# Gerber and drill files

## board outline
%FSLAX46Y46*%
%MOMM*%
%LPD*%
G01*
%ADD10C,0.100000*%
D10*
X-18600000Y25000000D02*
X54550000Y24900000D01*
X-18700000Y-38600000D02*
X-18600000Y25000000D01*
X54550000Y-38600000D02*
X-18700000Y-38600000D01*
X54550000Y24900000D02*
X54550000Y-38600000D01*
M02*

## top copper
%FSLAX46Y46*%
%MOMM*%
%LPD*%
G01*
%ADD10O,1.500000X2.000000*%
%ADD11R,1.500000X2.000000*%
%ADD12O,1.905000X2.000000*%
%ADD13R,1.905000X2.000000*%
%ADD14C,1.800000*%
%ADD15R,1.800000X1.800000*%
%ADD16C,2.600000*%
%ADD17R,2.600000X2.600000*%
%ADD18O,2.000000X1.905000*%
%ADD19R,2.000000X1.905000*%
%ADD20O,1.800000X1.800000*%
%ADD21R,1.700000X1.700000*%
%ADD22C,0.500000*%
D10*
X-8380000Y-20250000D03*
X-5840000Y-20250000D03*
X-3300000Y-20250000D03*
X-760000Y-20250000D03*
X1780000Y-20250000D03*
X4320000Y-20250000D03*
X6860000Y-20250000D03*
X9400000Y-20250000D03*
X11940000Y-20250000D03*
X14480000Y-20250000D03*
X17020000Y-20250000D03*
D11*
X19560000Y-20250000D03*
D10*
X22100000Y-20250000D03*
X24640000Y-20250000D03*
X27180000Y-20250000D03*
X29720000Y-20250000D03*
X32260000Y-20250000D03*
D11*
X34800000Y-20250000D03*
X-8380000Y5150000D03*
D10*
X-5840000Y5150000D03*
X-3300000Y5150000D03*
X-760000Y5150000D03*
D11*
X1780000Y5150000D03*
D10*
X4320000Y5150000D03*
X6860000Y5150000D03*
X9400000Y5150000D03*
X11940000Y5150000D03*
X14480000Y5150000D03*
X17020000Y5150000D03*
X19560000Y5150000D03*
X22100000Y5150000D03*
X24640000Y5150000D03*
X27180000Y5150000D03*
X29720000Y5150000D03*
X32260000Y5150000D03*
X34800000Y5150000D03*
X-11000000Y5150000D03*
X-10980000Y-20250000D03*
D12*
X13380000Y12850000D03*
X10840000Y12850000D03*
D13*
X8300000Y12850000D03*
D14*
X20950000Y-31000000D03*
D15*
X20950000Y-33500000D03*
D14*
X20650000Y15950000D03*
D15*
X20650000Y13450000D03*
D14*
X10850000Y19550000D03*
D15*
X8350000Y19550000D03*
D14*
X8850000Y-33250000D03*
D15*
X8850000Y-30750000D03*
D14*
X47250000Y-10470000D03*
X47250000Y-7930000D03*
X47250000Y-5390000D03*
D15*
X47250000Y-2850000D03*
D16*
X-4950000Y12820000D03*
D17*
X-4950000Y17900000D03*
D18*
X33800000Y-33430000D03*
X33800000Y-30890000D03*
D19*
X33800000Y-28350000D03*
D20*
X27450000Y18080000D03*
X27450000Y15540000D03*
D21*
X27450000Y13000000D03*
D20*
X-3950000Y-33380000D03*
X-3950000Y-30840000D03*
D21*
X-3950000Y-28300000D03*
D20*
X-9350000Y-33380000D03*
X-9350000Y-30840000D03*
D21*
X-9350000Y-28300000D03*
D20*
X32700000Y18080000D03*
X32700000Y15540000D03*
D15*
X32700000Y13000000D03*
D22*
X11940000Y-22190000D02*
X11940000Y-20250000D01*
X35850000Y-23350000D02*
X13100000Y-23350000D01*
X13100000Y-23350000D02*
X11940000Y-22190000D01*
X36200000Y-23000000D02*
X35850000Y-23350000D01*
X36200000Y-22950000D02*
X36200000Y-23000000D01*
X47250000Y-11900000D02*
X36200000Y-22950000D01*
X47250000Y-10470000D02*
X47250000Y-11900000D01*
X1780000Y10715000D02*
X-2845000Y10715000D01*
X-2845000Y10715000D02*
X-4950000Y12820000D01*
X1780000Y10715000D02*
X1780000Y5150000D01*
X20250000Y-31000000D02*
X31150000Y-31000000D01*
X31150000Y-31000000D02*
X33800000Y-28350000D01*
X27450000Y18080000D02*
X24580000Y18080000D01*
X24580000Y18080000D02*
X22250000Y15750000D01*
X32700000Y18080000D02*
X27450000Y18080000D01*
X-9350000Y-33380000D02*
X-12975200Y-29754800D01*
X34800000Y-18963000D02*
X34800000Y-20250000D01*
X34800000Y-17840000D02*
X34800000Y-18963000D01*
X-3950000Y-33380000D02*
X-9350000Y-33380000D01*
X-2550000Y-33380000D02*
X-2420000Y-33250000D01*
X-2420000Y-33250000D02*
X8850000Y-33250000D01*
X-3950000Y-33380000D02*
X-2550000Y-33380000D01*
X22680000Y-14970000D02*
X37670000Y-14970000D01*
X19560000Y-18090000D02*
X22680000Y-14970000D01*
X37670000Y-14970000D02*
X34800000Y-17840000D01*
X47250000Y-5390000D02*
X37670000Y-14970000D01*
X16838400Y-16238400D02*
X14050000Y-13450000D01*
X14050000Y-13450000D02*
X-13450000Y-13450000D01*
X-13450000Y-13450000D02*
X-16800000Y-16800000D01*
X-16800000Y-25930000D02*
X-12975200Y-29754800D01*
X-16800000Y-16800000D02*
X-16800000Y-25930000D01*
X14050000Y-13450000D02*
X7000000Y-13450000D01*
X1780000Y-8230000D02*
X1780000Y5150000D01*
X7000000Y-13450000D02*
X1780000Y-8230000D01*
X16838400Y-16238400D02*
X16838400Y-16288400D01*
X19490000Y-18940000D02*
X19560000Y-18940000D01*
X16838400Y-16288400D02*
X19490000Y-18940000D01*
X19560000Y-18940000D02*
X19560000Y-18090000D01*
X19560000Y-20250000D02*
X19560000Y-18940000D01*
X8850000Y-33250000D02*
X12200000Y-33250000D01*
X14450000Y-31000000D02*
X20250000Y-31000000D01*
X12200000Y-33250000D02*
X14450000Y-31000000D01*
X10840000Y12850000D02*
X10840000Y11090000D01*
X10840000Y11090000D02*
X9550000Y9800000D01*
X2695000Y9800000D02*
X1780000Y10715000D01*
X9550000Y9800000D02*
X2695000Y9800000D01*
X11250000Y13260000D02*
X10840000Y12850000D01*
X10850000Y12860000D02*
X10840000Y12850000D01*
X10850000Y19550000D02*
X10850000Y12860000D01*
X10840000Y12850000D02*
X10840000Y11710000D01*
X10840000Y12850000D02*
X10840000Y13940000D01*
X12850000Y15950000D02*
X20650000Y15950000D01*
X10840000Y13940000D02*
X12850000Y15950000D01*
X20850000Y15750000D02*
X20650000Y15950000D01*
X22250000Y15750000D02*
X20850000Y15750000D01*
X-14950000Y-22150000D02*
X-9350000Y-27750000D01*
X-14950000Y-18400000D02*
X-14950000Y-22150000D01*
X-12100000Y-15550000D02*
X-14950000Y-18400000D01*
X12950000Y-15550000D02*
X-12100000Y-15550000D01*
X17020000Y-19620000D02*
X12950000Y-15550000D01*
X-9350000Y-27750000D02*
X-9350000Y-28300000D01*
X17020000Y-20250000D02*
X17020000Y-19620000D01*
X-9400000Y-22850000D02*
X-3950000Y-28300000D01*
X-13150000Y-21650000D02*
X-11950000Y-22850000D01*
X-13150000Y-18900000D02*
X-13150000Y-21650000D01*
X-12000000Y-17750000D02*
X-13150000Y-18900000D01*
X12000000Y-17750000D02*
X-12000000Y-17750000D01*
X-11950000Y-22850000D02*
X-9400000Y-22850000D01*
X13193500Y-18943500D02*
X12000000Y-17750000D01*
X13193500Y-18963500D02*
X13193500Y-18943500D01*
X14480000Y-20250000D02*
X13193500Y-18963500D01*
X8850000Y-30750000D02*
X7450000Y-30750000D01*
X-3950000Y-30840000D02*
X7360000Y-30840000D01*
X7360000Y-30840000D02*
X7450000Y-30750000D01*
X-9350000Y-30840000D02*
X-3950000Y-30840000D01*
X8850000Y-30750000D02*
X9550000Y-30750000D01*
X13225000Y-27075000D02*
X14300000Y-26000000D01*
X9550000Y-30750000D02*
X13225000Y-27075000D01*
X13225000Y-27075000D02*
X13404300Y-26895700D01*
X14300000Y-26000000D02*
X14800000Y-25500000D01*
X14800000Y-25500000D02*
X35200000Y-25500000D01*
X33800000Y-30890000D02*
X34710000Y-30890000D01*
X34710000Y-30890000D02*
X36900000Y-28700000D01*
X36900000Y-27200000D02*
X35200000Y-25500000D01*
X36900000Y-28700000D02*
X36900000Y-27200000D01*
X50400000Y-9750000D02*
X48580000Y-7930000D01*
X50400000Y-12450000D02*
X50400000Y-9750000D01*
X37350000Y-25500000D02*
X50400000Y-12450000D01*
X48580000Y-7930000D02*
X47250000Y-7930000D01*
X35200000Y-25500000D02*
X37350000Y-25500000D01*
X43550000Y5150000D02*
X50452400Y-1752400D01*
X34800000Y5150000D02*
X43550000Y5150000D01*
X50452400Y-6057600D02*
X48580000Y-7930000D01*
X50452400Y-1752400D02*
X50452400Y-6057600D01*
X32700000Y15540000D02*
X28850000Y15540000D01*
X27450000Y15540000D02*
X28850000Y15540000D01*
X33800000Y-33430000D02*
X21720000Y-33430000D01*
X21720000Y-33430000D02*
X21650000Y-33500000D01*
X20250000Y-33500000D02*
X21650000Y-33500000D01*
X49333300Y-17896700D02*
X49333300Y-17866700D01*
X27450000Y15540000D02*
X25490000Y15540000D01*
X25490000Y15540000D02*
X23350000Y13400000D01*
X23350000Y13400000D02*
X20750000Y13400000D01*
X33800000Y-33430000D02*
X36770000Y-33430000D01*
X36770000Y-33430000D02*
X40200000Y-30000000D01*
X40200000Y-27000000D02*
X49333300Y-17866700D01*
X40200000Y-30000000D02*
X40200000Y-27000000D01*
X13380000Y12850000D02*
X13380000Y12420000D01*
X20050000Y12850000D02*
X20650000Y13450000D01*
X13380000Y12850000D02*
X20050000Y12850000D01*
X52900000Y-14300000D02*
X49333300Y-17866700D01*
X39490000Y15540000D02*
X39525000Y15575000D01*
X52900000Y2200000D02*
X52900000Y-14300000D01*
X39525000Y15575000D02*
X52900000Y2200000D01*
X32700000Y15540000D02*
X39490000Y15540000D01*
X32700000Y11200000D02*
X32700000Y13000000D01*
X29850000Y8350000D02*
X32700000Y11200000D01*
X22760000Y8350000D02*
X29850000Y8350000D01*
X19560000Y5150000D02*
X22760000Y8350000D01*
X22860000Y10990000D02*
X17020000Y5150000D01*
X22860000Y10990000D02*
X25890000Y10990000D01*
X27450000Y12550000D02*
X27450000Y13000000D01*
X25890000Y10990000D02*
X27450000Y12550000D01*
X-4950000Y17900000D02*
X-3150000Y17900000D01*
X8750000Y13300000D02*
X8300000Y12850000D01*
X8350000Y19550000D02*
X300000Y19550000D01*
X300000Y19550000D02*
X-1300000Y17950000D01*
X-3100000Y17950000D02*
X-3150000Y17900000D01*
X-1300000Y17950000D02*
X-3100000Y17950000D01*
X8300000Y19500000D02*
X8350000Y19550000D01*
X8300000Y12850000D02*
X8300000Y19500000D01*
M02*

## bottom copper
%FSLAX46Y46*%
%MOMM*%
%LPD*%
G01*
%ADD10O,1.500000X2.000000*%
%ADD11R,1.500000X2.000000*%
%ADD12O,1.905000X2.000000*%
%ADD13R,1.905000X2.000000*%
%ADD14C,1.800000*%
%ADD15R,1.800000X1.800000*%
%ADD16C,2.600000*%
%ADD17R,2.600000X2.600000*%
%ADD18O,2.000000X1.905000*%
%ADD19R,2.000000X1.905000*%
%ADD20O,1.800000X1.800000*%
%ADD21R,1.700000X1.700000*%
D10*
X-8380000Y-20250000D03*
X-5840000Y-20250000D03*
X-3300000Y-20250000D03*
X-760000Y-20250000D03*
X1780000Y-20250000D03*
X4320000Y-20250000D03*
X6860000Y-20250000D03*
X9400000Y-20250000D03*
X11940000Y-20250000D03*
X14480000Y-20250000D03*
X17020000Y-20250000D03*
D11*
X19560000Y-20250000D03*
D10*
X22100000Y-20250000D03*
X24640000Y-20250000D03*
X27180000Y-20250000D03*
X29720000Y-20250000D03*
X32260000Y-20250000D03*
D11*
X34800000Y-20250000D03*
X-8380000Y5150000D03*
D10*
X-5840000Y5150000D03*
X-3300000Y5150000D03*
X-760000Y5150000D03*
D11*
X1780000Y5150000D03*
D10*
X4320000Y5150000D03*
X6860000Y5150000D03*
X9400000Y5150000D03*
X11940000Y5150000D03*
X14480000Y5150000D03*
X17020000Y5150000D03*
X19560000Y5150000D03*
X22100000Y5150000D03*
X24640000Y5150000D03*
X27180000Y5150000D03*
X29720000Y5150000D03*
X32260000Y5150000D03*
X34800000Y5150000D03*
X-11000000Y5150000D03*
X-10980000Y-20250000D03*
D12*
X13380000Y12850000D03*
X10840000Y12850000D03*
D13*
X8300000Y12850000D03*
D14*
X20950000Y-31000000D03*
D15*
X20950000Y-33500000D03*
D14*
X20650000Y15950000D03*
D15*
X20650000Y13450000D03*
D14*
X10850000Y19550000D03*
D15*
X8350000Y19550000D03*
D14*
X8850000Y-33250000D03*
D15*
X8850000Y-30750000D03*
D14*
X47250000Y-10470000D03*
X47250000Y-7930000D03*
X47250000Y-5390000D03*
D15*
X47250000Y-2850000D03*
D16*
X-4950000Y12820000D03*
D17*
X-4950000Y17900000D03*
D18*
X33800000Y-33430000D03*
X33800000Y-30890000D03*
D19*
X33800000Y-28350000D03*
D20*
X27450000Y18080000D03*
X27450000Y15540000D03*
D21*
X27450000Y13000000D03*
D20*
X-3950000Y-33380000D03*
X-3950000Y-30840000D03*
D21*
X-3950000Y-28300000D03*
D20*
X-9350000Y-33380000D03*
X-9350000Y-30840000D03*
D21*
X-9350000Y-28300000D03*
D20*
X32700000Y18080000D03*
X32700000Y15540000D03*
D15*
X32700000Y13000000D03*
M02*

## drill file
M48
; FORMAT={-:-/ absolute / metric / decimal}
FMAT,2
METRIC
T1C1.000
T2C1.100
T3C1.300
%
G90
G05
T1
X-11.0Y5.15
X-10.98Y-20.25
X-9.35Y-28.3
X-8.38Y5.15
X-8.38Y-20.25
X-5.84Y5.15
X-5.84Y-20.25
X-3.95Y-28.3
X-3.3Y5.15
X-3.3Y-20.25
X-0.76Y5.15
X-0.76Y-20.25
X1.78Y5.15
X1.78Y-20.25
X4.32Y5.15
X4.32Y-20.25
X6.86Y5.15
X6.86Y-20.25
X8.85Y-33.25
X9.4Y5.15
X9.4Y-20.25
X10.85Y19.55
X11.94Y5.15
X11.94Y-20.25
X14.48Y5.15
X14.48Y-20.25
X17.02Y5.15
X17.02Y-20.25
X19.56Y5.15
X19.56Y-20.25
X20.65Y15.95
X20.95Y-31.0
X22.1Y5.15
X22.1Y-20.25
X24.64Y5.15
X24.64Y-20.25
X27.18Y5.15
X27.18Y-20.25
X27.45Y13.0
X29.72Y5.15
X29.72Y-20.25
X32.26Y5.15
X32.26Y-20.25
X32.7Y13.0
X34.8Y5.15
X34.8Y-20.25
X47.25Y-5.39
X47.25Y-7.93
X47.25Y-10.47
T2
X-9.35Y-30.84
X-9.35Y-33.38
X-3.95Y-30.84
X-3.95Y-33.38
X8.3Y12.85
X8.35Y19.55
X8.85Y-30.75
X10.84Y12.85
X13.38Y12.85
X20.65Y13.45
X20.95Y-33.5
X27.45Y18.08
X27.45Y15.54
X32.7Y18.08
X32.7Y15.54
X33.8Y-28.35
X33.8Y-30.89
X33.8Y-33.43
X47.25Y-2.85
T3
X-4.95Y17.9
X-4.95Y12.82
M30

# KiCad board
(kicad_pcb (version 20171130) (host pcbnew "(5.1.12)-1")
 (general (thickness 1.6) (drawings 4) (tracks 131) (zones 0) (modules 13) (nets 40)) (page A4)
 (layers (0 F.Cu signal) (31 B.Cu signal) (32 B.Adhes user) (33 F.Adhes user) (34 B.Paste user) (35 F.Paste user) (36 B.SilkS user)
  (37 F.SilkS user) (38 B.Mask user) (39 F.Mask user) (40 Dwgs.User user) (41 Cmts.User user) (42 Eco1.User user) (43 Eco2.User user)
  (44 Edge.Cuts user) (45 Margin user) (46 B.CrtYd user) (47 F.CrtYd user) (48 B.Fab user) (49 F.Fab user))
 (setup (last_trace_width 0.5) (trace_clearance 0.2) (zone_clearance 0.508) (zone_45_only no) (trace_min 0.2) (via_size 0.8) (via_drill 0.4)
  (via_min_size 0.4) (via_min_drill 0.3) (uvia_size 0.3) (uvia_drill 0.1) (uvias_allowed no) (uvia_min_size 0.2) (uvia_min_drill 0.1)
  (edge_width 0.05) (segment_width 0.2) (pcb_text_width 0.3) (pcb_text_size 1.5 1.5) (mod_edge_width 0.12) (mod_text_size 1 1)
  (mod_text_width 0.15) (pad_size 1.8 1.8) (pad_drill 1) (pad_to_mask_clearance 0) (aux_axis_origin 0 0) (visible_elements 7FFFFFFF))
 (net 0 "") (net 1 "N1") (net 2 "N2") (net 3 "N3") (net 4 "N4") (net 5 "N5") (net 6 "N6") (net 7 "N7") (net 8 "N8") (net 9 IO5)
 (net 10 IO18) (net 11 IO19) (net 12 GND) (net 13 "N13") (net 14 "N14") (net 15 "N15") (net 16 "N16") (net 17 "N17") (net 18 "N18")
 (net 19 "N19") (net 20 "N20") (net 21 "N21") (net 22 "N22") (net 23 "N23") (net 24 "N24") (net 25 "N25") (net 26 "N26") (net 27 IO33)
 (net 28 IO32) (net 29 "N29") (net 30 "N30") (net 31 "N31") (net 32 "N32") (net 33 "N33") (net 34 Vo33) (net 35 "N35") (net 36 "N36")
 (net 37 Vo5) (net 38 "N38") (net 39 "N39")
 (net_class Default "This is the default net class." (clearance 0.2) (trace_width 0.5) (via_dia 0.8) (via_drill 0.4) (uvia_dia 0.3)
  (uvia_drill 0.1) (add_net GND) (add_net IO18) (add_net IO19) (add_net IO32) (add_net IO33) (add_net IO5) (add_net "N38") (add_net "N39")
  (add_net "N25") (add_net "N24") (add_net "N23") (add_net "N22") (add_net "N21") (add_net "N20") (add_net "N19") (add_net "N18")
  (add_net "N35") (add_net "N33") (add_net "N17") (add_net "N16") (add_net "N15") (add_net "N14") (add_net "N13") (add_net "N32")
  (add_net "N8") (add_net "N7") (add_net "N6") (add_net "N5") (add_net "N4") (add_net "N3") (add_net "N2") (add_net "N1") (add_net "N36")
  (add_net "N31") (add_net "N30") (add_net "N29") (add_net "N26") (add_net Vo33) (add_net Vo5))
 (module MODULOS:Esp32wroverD (layer F.Cu) (at 12.4 7.55)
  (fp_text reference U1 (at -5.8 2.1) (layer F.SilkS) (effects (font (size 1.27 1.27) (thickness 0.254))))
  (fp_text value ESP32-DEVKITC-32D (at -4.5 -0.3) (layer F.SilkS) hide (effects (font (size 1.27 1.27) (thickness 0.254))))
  (pad 37 thru_hole oval (at -20.78 12.7) (size 1.5 2) (drill 1) (layers *.Cu *.Mask) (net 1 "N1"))
  (pad 36 thru_hole oval (at -18.24 12.7) (size 1.5 2) (drill 1) (layers *.Cu *.Mask) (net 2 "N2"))
  (pad 35 thru_hole oval (at -15.7 12.7) (size 1.5 2) (drill 1) (layers *.Cu *.Mask) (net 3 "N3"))
  (pad 34 thru_hole oval (at -13.16 12.7) (size 1.5 2) (drill 1) (layers *.Cu *.Mask) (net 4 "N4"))
  (pad 33 thru_hole oval (at -10.62 12.7) (size 1.5 2) (drill 1) (layers *.Cu *.Mask) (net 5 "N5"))
  (pad 32 thru_hole oval (at -8.08 12.7) (size 1.5 2) (drill 1) (layers *.Cu *.Mask) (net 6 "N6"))
  (pad 31 thru_hole oval (at -5.54 12.7) (size 1.5 2) (drill 1) (layers *.Cu *.Mask) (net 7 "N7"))
  (pad 30 thru_hole oval (at -3 12.7) (size 1.5 2) (drill 1) (layers *.Cu *.Mask) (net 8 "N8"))
  (pad 29 thru_hole oval (at -0.46 12.7) (size 1.5 2) (drill 1) (layers *.Cu *.Mask) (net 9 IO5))
  (pad 28 thru_hole oval (at 2.08 12.7) (size 1.5 2) (drill 1) (layers *.Cu *.Mask) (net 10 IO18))
  (pad 27 thru_hole oval (at 4.62 12.7) (size 1.5 2) (drill 1) (layers *.Cu *.Mask) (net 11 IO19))
  (pad 26 thru_hole rect (at 7.16 12.7) (size 1.5 2) (drill 1) (layers *.Cu *.Mask) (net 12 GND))
  (pad 25 thru_hole oval (at 9.7 12.7) (size 1.5 2) (drill 1) (layers *.Cu *.Mask) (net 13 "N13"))
  (pad 24 thru_hole oval (at 12.24 12.7) (size 1.5 2) (drill 1) (layers *.Cu *.Mask) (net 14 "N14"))
  (pad 23 thru_hole oval (at 14.78 12.7) (size 1.5 2) (drill 1) (layers *.Cu *.Mask) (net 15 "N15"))
  (pad 22 thru_hole oval (at 17.32 12.7) (size 1.5 2) (drill 1) (layers *.Cu *.Mask) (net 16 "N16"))
  (pad 21 thru_hole oval (at 19.86 12.7) (size 1.5 2) (drill 1) (layers *.Cu *.Mask) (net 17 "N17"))
  (pad 20 thru_hole rect (at 22.4 12.7) (size 1.5 2) (drill 1) (layers *.Cu *.Mask) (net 12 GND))
  (pad 18 thru_hole rect (at -20.78 -12.7) (size 1.5 2) (drill 1) (layers *.Cu *.Mask) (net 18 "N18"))
  (pad 17 thru_hole oval (at -18.24 -12.7) (size 1.5 2) (drill 1) (layers *.Cu *.Mask) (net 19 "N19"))
  (pad 16 thru_hole oval (at -15.7 -12.7) (size 1.5 2) (drill 1) (layers *.Cu *.Mask) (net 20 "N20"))
  (pad 15 thru_hole oval (at -13.16 -12.7) (size 1.5 2) (drill 1) (layers *.Cu *.Mask) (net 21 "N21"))
  (pad 14 thru_hole rect (at -10.62 -12.7) (size 1.5 2) (drill 1) (layers *.Cu *.Mask) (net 12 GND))
  (pad 13 thru_hole oval (at -8.08 -12.7) (size 1.5 2) (drill 1) (layers *.Cu *.Mask) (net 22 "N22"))
  (pad 12 thru_hole oval (at -5.54 -12.7) (size 1.5 2) (drill 1) (layers *.Cu *.Mask) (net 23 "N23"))
  (pad 11 thru_hole oval (at -3 -12.7) (size 1.5 2) (drill 1) (layers *.Cu *.Mask) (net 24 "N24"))
  (pad 10 thru_hole oval (at -0.46 -12.7) (size 1.5 2) (drill 1) (layers *.Cu *.Mask) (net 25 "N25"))
  (pad 9 thru_hole oval (at 2.08 -12.7) (size 1.5 2) (drill 1) (layers *.Cu *.Mask) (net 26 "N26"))
  (pad 8 thru_hole oval (at 4.62 -12.7) (size 1.5 2) (drill 1) (layers *.Cu *.Mask) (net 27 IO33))
  (pad 7 thru_hole oval (at 7.16 -12.7) (size 1.5 2) (drill 1) (layers *.Cu *.Mask) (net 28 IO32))
  (pad 6 thru_hole oval (at 9.7 -12.7) (size 1.5 2) (drill 1) (layers *.Cu *.Mask) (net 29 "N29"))
  (pad 5 thru_hole oval (at 12.24 -12.7) (size 1.5 2) (drill 1) (layers *.Cu *.Mask) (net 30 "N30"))
  (pad 4 thru_hole oval (at 14.78 -12.7) (size 1.5 2) (drill 1) (layers *.Cu *.Mask) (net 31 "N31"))
  (pad 3 thru_hole oval (at 17.32 -12.7) (size 1.5 2) (drill 1) (layers *.Cu *.Mask) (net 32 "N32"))
  (pad 2 thru_hole oval (at 19.86 -12.7) (size 1.5 2) (drill 1) (layers *.Cu *.Mask) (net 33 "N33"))
  (pad 1 thru_hole oval (at 22.4 -12.7) (size 1.5 2) (drill 1) (layers *.Cu *.Mask) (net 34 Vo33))
  (pad 19 thru_hole oval (at -23.4 -12.7) (size 1.5 2) (drill 1) (layers *.Cu *.Mask) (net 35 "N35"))
  (pad 38 thru_hole oval (at -23.38 12.7) (size 1.5 2) (drill 1) (layers *.Cu *.Mask) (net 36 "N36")))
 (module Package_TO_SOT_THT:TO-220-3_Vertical (layer F.Cu) (at 8.3 -12.85)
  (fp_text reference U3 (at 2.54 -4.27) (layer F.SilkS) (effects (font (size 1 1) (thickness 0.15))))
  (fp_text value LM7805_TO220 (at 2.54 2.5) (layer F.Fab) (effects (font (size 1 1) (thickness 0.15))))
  (pad 3 thru_hole oval (at 5.08 0) (size 1.905 2) (drill 1.1) (layers *.Cu *.Mask) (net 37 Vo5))
  (pad 2 thru_hole oval (at 2.54 0) (size 1.905 2) (drill 1.1) (layers *.Cu *.Mask) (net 12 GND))
  (pad 1 thru_hole rect (at 0 0) (size 1.905 2) (drill 1.1) (layers *.Cu *.Mask) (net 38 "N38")))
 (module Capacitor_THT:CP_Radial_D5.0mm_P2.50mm (layer F.Cu) (at 20.95 33.5 90)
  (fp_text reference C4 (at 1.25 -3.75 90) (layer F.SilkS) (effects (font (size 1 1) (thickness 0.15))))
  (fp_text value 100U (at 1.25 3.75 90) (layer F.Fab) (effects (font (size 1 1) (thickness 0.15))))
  (pad 2 thru_hole circle (at 2.5 0 90) (size 1.8 1.8) (drill 1) (layers *.Cu *.Mask) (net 12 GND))
  (pad 1 thru_hole rect (at 0 0 90) (size 1.8 1.8) (drill 1.1) (layers *.Cu *.Mask) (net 37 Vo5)))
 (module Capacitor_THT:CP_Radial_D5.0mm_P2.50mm (layer F.Cu) (at 20.65 -13.45 90)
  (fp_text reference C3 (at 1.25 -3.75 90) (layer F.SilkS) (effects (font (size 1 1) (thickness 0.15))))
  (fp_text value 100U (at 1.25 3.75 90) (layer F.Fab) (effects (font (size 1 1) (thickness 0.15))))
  (pad 2 thru_hole circle (at 2.5 0 90) (size 1.8 1.8) (drill 1) (layers *.Cu *.Mask) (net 12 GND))
  (pad 1 thru_hole rect (at 0 0 90) (size 1.8 1.8) (drill 1.1) (layers *.Cu *.Mask) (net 37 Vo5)))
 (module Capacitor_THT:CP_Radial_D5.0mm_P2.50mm (layer F.Cu) (at 8.35 -19.55)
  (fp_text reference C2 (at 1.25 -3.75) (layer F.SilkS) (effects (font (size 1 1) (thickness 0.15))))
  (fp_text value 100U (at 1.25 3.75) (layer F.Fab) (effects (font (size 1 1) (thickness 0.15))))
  (pad 2 thru_hole circle (at 2.5 0) (size 1.8 1.8) (drill 1) (layers *.Cu *.Mask) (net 12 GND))
  (pad 1 thru_hole rect (at 0 0) (size 1.8 1.8) (drill 1.1) (layers *.Cu *.Mask) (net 38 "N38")))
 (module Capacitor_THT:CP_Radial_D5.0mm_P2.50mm (layer F.Cu) (at 8.85 30.75 270)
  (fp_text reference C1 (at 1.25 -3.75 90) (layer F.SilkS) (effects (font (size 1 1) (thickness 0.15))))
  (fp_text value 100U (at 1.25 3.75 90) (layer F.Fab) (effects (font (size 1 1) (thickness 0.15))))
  (pad 2 thru_hole circle (at 2.5 0 270) (size 1.8 1.8) (drill 1) (layers *.Cu *.Mask) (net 12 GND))
  (pad 1 thru_hole rect (at 0 0 270) (size 1.8 1.8) (drill 1.1) (layers *.Cu *.Mask) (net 34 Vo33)))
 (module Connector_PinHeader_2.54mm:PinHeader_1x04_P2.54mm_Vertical (layer F.Cu) (at 47.25 2.85)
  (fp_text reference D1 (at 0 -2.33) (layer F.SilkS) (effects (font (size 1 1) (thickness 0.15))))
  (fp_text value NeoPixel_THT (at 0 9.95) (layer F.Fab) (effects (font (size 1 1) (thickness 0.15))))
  (pad 4 thru_hole circle (at 0 7.62) (size 1.8 1.8) (drill 1) (layers *.Cu *.Mask) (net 9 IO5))
  (pad 3 thru_hole circle (at 0 5.08) (size 1.8 1.8) (drill 1) (layers *.Cu *.Mask) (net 34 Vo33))
  (pad 2 thru_hole circle (at 0 2.54) (size 1.8 1.8) (drill 1) (layers *.Cu *.Mask) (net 12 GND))
  (pad 1 thru_hole rect (at 0 0) (size 1.8 1.8) (drill 1.1) (layers *.Cu *.Mask) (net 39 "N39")))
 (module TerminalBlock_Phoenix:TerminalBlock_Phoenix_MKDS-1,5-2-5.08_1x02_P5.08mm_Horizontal (layer F.Cu) (at -4.95 -17.9 270)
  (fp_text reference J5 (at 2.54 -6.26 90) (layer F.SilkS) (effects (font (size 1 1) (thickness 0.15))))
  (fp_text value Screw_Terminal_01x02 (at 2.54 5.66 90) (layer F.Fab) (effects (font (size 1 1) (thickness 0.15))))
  (pad 2 thru_hole circle (at 5.08 0 270) (size 2.6 2.6) (drill 1.3) (layers *.Cu *.Mask) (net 12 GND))
  (pad 1 thru_hole rect (at 0 0 270) (size 2.6 2.6) (drill 1.3) (layers *.Cu *.Mask) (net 38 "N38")))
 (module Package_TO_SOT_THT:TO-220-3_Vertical (layer F.Cu) (at 33.8 28.35 270)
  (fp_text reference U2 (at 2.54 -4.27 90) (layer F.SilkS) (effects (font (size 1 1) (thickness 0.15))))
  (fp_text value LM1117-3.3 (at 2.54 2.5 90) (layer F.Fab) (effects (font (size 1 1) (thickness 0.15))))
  (pad 3 thru_hole oval (at 5.08 0 270) (size 1.905 2) (drill 1.1) (layers *.Cu *.Mask) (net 37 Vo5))
  (pad 2 thru_hole oval (at 2.54 0 270) (size 1.905 2) (drill 1.1) (layers *.Cu *.Mask) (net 34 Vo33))
  (pad 1 thru_hole rect (at 0 0 270) (size 1.905 2) (drill 1.1) (layers *.Cu *.Mask) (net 12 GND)))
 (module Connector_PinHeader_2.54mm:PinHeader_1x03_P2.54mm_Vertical (layer F.Cu) (at 27.45 -13 180)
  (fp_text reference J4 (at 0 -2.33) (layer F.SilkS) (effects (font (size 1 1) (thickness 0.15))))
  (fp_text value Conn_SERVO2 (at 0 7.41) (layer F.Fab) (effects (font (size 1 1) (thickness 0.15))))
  (pad 3 thru_hole oval (at 0 5.08 180) (size 1.8 1.8) (drill 1.1) (layers *.Cu *.Mask) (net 12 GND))
  (pad 2 thru_hole oval (at 0 2.54 180) (size 1.8 1.8) (drill 1.1) (layers *.Cu *.Mask) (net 37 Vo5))
  (pad 1 thru_hole rect (at 0 0 180) (size 1.7 1.7) (drill 1) (layers *.Cu *.Mask) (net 27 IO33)))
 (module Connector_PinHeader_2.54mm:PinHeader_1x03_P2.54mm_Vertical (layer F.Cu) (at -3.95 28.3)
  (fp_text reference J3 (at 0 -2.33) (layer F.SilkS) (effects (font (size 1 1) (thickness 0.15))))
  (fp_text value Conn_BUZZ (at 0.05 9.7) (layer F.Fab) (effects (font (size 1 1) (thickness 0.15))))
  (pad 3 thru_hole oval (at 0 5.08) (size 1.8 1.8) (drill 1.1) (layers *.Cu *.Mask) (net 12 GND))
  (pad 2 thru_hole oval (at 0 2.54) (size 1.8 1.8) (drill 1.1) (layers *.Cu *.Mask) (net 34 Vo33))
  (pad 1 thru_hole rect (at 0 0) (size 1.7 1.7) (drill 1) (layers *.Cu *.Mask) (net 10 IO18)))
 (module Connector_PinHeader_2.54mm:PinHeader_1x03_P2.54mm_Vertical (layer F.Cu) (at -9.35 28.3)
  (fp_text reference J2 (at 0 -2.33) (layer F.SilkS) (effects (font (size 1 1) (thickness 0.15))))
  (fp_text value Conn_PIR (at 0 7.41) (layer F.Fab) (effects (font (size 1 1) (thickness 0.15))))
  (pad 3 thru_hole oval (at 0 5.08) (size 1.8 1.8) (drill 1.1) (layers *.Cu *.Mask) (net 12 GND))
  (pad 2 thru_hole oval (at 0 2.54) (size 1.8 1.8) (drill 1.1) (layers *.Cu *.Mask) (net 34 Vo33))
  (pad 1 thru_hole rect (at 0 0) (size 1.7 1.7) (drill 1) (layers *.Cu *.Mask) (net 11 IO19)))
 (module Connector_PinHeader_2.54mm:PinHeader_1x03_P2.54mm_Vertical (layer F.Cu) (at 32.7 -13 180)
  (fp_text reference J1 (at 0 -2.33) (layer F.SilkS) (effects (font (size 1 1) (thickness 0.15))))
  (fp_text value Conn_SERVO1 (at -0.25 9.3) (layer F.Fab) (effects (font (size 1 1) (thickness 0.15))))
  (pad 3 thru_hole oval (at 0 5.08 180) (size 1.8 1.8) (drill 1.1) (layers *.Cu *.Mask) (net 12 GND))
  (pad 2 thru_hole oval (at 0 2.54 180) (size 1.8 1.8) (drill 1.1) (layers *.Cu *.Mask) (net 37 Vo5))
  (pad 1 thru_hole rect (at 0 0 180) (size 1.8 1.8) (drill 1) (layers *.Cu *.Mask) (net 28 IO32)))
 (gr_line (start -18.6 -25) (end 54.55 -24.9) (layer Edge.Cuts) (width 0.1))
 (gr_line (start -18.7 38.6) (end -18.6 -25) (layer Edge.Cuts) (width 0.1))
 (gr_line (start 54.55 38.6) (end -18.7 38.6) (layer Edge.Cuts) (width 0.1))
 (gr_line (start 54.55 -24.9) (end 54.55 38.6) (layer Edge.Cuts) (width 0.1))
 (segment (start 11.94 22.19) (end 11.94 20.25) (width 0.5) (layer F.Cu) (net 9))
 (segment (start 35.85 23.35) (end 13.1 23.35) (width 0.5) (layer F.Cu) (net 9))
 (segment (start 13.1 23.35) (end 11.94 22.19) (width 0.5) (layer F.Cu) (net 9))
 (segment (start 36.2 23) (end 35.85 23.35) (width 0.5) (layer F.Cu) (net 9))
 (segment (start 36.2 22.95) (end 36.2 23) (width 0.5) (layer F.Cu) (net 9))
 (segment (start 47.25 11.9) (end 36.2 22.95) (width 0.5) (layer F.Cu) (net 9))
 (segment (start 47.25 10.47) (end 47.25 11.9) (width 0.5) (layer F.Cu) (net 9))
 (segment (start 1.78 -10.715) (end -2.845 -10.715) (width 0.5) (layer F.Cu) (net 12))
 (segment (start -2.845 -10.715) (end -4.95 -12.82) (width 0.5) (layer F.Cu) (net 12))
 (segment (start 1.78 -10.715) (end 1.78 -5.15) (width 0.5) (layer F.Cu) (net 12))
 (segment (start 20.25 31) (end 31.15 31) (width 0.5) (layer F.Cu) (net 12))
 (segment (start 31.15 31) (end 33.8 28.35) (width 0.5) (layer F.Cu) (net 12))
 (segment (start 27.45 -18.08) (end 24.58 -18.08) (width 0.5) (layer F.Cu) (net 12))
 (segment (start 24.58 -18.08) (end 22.25 -15.75) (width 0.5) (layer F.Cu) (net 12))
 (segment (start 32.7 -18.08) (end 27.45 -18.08) (width 0.5) (layer F.Cu) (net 12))
 (segment (start -9.35 33.38) (end -12.9752 29.7548) (width 0.5) (layer F.Cu) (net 12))
 (segment (start 34.8 18.963) (end 34.8 20.25) (width 0.5) (layer F.Cu) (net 12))
 (segment (start 34.8 17.84) (end 34.8 18.963) (width 0.5) (layer F.Cu) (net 12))
 (segment (start -3.95 33.38) (end -9.35 33.38) (width 0.5) (layer F.Cu) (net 12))
 (segment (start -2.55 33.38) (end -2.42 33.25) (width 0.5) (layer F.Cu) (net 12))
 (segment (start -2.42 33.25) (end 8.85 33.25) (width 0.5) (layer F.Cu) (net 12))
 (segment (start -3.95 33.38) (end -2.55 33.38) (width 0.5) (layer F.Cu) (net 12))
 (segment (start 22.68 14.97) (end 37.67 14.97) (width 0.5) (layer F.Cu) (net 12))
 (segment (start 19.56 18.09) (end 22.68 14.97) (width 0.5) (layer F.Cu) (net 12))
 (segment (start 37.67 14.97) (end 34.8 17.84) (width 0.5) (layer F.Cu) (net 12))
 (segment (start 47.25 5.39) (end 37.67 14.97) (width 0.5) (layer F.Cu) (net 12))
 (segment (start 16.8384 16.2384) (end 14.05 13.45) (width 0.5) (layer F.Cu) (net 12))
 (segment (start 14.05 13.45) (end -13.45 13.45) (width 0.5) (layer F.Cu) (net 12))
 (segment (start -13.45 13.45) (end -16.8 16.8) (width 0.5) (layer F.Cu) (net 12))
 (segment (start -16.8 25.93) (end -12.9752 29.7548) (width 0.5) (layer F.Cu) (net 12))
 (segment (start -16.8 16.8) (end -16.8 25.93) (width 0.5) (layer F.Cu) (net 12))
 (segment (start 14.05 13.45) (end 7 13.45) (width 0.5) (layer F.Cu) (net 12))
 (segment (start 1.78 8.23) (end 1.78 -5.15) (width 0.5) (layer F.Cu) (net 12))
 (segment (start 7 13.45) (end 1.78 8.23) (width 0.5) (layer F.Cu) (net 12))
 (segment (start 16.8384 16.2384) (end 16.8384 16.2884) (width 0.5) (layer F.Cu) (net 12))
 (segment (start 19.49 18.94) (end 19.56 18.94) (width 0.5) (layer F.Cu) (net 12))
 (segment (start 16.8384 16.2884) (end 19.49 18.94) (width 0.5) (layer F.Cu) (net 12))
 (segment (start 19.56 18.94) (end 19.56 18.09) (width 0.5) (layer F.Cu) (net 12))
 (segment (start 19.56 20.25) (end 19.56 18.94) (width 0.5) (layer F.Cu) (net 12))
 (segment (start 8.85 33.25) (end 12.2 33.25) (width 0.5) (layer F.Cu) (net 12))
 (segment (start 14.45 31) (end 20.25 31) (width 0.5) (layer F.Cu) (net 12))
 (segment (start 12.2 33.25) (end 14.45 31) (width 0.5) (layer F.Cu) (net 12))
 (segment (start 10.84 -12.85) (end 10.84 -11.09) (width 0.5) (layer F.Cu) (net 12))
 (segment (start 10.84 -11.09) (end 9.55 -9.8) (width 0.5) (layer F.Cu) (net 12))
 (segment (start 2.695 -9.8) (end 1.78 -10.715) (width 0.5) (layer F.Cu) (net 12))
 (segment (start 9.55 -9.8) (end 2.695 -9.8) (width 0.5) (layer F.Cu) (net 12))
 (segment (start 11.25 -13.26) (end 10.84 -12.85) (width 0.5) (layer F.Cu) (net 12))
 (segment (start 10.85 -12.86) (end 10.84 -12.85) (width 0.5) (layer F.Cu) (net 12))
 (segment (start 10.85 -19.55) (end 10.85 -12.86) (width 0.5) (layer F.Cu) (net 12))
 (segment (start 10.84 -12.85) (end 10.84 -11.71) (width 0.5) (layer F.Cu) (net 12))
 (segment (start 10.84 -12.85) (end 10.84 -13.94) (width 0.5) (layer F.Cu) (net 12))
 (segment (start 12.85 -15.95) (end 20.65 -15.95) (width 0.5) (layer F.Cu) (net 12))
 (segment (start 10.84 -13.94) (end 12.85 -15.95) (width 0.5) (layer F.Cu) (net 12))
 (segment (start 20.85 -15.75) (end 20.65 -15.95) (width 0.5) (layer F.Cu) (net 12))
 (segment (start 22.25 -15.75) (end 20.85 -15.75) (width 0.5) (layer F.Cu) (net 12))
 (segment (start -14.95 22.15) (end -9.35 27.75) (width 0.5) (layer F.Cu) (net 11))
 (segment (start -14.95 18.4) (end -14.95 22.15) (width 0.5) (layer F.Cu) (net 11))
 (segment (start -12.1 15.55) (end -14.95 18.4) (width 0.5) (layer F.Cu) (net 11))
 (segment (start 12.95 15.55) (end -12.1 15.55) (width 0.5) (layer F.Cu) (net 11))
 (segment (start 17.02 19.62) (end 12.95 15.55) (width 0.5) (layer F.Cu) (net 11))
 (segment (start -9.35 27.75) (end -9.35 28.3) (width 0.5) (layer F.Cu) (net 11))
 (segment (start 17.02 20.25) (end 17.02 19.62) (width 0.5) (layer F.Cu) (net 11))
 (segment (start -9.4 22.85) (end -3.95 28.3) (width 0.5) (layer F.Cu) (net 10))
 (segment (start -13.15 21.65) (end -11.95 22.85) (width 0.5) (layer F.Cu) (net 10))
 (segment (start -13.15 18.9) (end -13.15 21.65) (width 0.5) (layer F.Cu) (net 10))
 (segment (start -12 17.75) (end -13.15 18.9) (width 0.5) (layer F.Cu) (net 10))
 (segment (start 12 17.75) (end -12 17.75) (width 0.5) (layer F.Cu) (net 10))
 (segment (start -11.95 22.85) (end -9.4 22.85) (width 0.5) (layer F.Cu) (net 10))
 (segment (start 13.1935 18.9435) (end 12 17.75) (width 0.5) (layer F.Cu) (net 10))
 (segment (start 13.1935 18.9635) (end 13.1935 18.9435) (width 0.5) (layer F.Cu) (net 10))
 (segment (start 14.48 20.25) (end 13.1935 18.9635) (width 0.5) (layer F.Cu) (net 10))
 (segment (start 8.85 30.75) (end 7.45 30.75) (width 0.5) (layer F.Cu) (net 34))
 (segment (start -3.95 30.84) (end 7.36 30.84) (width 0.5) (layer F.Cu) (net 34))
 (segment (start 7.36 30.84) (end 7.45 30.75) (width 0.5) (layer F.Cu) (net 34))
 (segment (start -9.35 30.84) (end -3.95 30.84) (width 0.5) (layer F.Cu) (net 34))
 (segment (start 8.85 30.75) (end 9.55 30.75) (width 0.5) (layer F.Cu) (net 34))
 (segment (start 13.225 27.075) (end 14.3 26) (width 0.5) (layer F.Cu) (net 34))
 (segment (start 9.55 30.75) (end 13.225 27.075) (width 0.5) (layer F.Cu) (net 34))
 (segment (start 13.225 27.075) (end 13.4043 26.8957) (width 0.5) (layer F.Cu) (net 34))
 (segment (start 14.3 26) (end 14.8 25.5) (width 0.5) (layer F.Cu) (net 34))
 (segment (start 14.8 25.5) (end 35.2 25.5) (width 0.5) (layer F.Cu) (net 34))
 (segment (start 33.8 30.89) (end 34.71 30.89) (width 0.5) (layer F.Cu) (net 34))
 (segment (start 34.71 30.89) (end 36.9 28.7) (width 0.5) (layer F.Cu) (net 34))
 (segment (start 36.9 27.2) (end 35.2 25.5) (width 0.5) (layer F.Cu) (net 34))
 (segment (start 36.9 28.7) (end 36.9 27.2) (width 0.5) (layer F.Cu) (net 34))
 (segment (start 50.4 9.75) (end 48.58 7.93) (width 0.5) (layer F.Cu) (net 34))
 (segment (start 50.4 12.45) (end 50.4 9.75) (width 0.5) (layer F.Cu) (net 34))
 (segment (start 37.35 25.5) (end 50.4 12.45) (width 0.5) (layer F.Cu) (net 34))
 (segment (start 48.58 7.93) (end 47.25 7.93) (width 0.5) (layer F.Cu) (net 34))
 (segment (start 35.2 25.5) (end 37.35 25.5) (width 0.5) (layer F.Cu) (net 34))
 (segment (start 43.55 -5.15) (end 50.4524 1.7524) (width 0.5) (layer F.Cu) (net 34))
 (segment (start 34.8 -5.15) (end 43.55 -5.15) (width 0.5) (layer F.Cu) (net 34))
 (segment (start 50.4524 6.0576) (end 48.58 7.93) (width 0.5) (layer F.Cu) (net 34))
 (segment (start 50.4524 1.7524) (end 50.4524 6.0576) (width 0.5) (layer F.Cu) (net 34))
 (segment (start 32.7 -15.54) (end 28.85 -15.54) (width 0.5) (layer F.Cu) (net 37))
 (segment (start 27.45 -15.54) (end 28.85 -15.54) (width 0.5) (layer F.Cu) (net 37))
 (segment (start 33.8 33.43) (end 21.72 33.43) (width 0.5) (layer F.Cu) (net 37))
 (segment (start 21.72 33.43) (end 21.65 33.5) (width 0.5) (layer F.Cu) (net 37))
 (segment (start 20.25 33.5) (end 21.65 33.5) (width 0.5) (layer F.Cu) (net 37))
 (segment (start 49.3333 17.8967) (end 49.3333 17.8667) (width 0.5) (layer F.Cu) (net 37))
 (segment (start 27.45 -15.54) (end 25.49 -15.54) (width 0.5) (layer F.Cu) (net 37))
 (segment (start 25.49 -15.54) (end 23.35 -13.4) (width 0.5) (layer F.Cu) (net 37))
 (segment (start 23.35 -13.4) (end 20.75 -13.4) (width 0.5) (layer F.Cu) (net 37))
 (segment (start 33.8 33.43) (end 36.77 33.43) (width 0.5) (layer F.Cu) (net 37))
 (segment (start 36.77 33.43) (end 40.2 30) (width 0.5) (layer F.Cu) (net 37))
 (segment (start 40.2 27) (end 49.3333 17.8667) (width 0.5) (layer F.Cu) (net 37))
 (segment (start 40.2 30) (end 40.2 27) (width 0.5) (layer F.Cu) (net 37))
 (segment (start 13.38 -12.85) (end 13.38 -12.42) (width 0.5) (layer F.Cu) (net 37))
 (segment (start 20.05 -12.85) (end 20.65 -13.45) (width 0.5) (layer F.Cu) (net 37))
 (segment (start 13.38 -12.85) (end 20.05 -12.85) (width 0.5) (layer F.Cu) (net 37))
 (segment (start 52.9 14.3) (end 49.3333 17.8667) (width 0.5) (layer F.Cu) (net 37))
 (segment (start 39.49 -15.54) (end 39.525 -15.575) (width 0.5) (layer F.Cu) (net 37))
 (segment (start 52.9 -2.2) (end 52.9 14.3) (width 0.5) (layer F.Cu) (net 37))
 (segment (start 39.525 -15.575) (end 52.9 -2.2) (width 0.5) (layer F.Cu) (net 37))
 (segment (start 32.7 -15.54) (end 39.49 -15.54) (width 0.5) (layer F.Cu) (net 37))
 (segment (start 32.7 -11.2) (end 32.7 -13) (width 0.5) (layer F.Cu) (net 28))
 (segment (start 29.85 -8.35) (end 32.7 -11.2) (width 0.5) (layer F.Cu) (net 28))
 (segment (start 22.76 -8.35) (end 29.85 -8.35) (width 0.5) (layer F.Cu) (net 28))
 (segment (start 19.56 -5.15) (end 22.76 -8.35) (width 0.5) (layer F.Cu) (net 28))
 (segment (start 22.86 -10.99) (end 17.02 -5.15) (width 0.5) (layer F.Cu) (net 27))
 (segment (start 22.86 -10.99) (end 25.89 -10.99) (width 0.5) (layer F.Cu) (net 27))
 (segment (start 27.45 -12.55) (end 27.45 -13) (width 0.5) (layer F.Cu) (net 27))
 (segment (start 25.89 -10.99) (end 27.45 -12.55) (width 0.5) (layer F.Cu) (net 27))
 (segment (start -4.95 -17.9) (end -3.15 -17.9) (width 0.5) (layer F.Cu) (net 38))
 (segment (start 8.75 -13.3) (end 8.3 -12.85) (width 0.5) (layer F.Cu) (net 38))
 (segment (start 8.35 -19.55) (end 0.3 -19.55) (width 0.5) (layer F.Cu) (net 38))
 (segment (start 0.3 -19.55) (end -1.3 -17.95) (width 0.5) (layer F.Cu) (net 38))
 (segment (start -3.1 -17.95) (end -3.15 -17.9) (width 0.5) (layer F.Cu) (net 38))
 (segment (start -1.3 -17.95) (end -3.1 -17.95) (width 0.5) (layer F.Cu) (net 38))
 (segment (start 8.3 -19.5) (end 8.35 -19.55) (width 0.5) (layer F.Cu) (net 38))
 (segment (start 8.3 -12.85) (end 8.3 -19.5) (width 0.5) (layer F.Cu) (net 38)))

